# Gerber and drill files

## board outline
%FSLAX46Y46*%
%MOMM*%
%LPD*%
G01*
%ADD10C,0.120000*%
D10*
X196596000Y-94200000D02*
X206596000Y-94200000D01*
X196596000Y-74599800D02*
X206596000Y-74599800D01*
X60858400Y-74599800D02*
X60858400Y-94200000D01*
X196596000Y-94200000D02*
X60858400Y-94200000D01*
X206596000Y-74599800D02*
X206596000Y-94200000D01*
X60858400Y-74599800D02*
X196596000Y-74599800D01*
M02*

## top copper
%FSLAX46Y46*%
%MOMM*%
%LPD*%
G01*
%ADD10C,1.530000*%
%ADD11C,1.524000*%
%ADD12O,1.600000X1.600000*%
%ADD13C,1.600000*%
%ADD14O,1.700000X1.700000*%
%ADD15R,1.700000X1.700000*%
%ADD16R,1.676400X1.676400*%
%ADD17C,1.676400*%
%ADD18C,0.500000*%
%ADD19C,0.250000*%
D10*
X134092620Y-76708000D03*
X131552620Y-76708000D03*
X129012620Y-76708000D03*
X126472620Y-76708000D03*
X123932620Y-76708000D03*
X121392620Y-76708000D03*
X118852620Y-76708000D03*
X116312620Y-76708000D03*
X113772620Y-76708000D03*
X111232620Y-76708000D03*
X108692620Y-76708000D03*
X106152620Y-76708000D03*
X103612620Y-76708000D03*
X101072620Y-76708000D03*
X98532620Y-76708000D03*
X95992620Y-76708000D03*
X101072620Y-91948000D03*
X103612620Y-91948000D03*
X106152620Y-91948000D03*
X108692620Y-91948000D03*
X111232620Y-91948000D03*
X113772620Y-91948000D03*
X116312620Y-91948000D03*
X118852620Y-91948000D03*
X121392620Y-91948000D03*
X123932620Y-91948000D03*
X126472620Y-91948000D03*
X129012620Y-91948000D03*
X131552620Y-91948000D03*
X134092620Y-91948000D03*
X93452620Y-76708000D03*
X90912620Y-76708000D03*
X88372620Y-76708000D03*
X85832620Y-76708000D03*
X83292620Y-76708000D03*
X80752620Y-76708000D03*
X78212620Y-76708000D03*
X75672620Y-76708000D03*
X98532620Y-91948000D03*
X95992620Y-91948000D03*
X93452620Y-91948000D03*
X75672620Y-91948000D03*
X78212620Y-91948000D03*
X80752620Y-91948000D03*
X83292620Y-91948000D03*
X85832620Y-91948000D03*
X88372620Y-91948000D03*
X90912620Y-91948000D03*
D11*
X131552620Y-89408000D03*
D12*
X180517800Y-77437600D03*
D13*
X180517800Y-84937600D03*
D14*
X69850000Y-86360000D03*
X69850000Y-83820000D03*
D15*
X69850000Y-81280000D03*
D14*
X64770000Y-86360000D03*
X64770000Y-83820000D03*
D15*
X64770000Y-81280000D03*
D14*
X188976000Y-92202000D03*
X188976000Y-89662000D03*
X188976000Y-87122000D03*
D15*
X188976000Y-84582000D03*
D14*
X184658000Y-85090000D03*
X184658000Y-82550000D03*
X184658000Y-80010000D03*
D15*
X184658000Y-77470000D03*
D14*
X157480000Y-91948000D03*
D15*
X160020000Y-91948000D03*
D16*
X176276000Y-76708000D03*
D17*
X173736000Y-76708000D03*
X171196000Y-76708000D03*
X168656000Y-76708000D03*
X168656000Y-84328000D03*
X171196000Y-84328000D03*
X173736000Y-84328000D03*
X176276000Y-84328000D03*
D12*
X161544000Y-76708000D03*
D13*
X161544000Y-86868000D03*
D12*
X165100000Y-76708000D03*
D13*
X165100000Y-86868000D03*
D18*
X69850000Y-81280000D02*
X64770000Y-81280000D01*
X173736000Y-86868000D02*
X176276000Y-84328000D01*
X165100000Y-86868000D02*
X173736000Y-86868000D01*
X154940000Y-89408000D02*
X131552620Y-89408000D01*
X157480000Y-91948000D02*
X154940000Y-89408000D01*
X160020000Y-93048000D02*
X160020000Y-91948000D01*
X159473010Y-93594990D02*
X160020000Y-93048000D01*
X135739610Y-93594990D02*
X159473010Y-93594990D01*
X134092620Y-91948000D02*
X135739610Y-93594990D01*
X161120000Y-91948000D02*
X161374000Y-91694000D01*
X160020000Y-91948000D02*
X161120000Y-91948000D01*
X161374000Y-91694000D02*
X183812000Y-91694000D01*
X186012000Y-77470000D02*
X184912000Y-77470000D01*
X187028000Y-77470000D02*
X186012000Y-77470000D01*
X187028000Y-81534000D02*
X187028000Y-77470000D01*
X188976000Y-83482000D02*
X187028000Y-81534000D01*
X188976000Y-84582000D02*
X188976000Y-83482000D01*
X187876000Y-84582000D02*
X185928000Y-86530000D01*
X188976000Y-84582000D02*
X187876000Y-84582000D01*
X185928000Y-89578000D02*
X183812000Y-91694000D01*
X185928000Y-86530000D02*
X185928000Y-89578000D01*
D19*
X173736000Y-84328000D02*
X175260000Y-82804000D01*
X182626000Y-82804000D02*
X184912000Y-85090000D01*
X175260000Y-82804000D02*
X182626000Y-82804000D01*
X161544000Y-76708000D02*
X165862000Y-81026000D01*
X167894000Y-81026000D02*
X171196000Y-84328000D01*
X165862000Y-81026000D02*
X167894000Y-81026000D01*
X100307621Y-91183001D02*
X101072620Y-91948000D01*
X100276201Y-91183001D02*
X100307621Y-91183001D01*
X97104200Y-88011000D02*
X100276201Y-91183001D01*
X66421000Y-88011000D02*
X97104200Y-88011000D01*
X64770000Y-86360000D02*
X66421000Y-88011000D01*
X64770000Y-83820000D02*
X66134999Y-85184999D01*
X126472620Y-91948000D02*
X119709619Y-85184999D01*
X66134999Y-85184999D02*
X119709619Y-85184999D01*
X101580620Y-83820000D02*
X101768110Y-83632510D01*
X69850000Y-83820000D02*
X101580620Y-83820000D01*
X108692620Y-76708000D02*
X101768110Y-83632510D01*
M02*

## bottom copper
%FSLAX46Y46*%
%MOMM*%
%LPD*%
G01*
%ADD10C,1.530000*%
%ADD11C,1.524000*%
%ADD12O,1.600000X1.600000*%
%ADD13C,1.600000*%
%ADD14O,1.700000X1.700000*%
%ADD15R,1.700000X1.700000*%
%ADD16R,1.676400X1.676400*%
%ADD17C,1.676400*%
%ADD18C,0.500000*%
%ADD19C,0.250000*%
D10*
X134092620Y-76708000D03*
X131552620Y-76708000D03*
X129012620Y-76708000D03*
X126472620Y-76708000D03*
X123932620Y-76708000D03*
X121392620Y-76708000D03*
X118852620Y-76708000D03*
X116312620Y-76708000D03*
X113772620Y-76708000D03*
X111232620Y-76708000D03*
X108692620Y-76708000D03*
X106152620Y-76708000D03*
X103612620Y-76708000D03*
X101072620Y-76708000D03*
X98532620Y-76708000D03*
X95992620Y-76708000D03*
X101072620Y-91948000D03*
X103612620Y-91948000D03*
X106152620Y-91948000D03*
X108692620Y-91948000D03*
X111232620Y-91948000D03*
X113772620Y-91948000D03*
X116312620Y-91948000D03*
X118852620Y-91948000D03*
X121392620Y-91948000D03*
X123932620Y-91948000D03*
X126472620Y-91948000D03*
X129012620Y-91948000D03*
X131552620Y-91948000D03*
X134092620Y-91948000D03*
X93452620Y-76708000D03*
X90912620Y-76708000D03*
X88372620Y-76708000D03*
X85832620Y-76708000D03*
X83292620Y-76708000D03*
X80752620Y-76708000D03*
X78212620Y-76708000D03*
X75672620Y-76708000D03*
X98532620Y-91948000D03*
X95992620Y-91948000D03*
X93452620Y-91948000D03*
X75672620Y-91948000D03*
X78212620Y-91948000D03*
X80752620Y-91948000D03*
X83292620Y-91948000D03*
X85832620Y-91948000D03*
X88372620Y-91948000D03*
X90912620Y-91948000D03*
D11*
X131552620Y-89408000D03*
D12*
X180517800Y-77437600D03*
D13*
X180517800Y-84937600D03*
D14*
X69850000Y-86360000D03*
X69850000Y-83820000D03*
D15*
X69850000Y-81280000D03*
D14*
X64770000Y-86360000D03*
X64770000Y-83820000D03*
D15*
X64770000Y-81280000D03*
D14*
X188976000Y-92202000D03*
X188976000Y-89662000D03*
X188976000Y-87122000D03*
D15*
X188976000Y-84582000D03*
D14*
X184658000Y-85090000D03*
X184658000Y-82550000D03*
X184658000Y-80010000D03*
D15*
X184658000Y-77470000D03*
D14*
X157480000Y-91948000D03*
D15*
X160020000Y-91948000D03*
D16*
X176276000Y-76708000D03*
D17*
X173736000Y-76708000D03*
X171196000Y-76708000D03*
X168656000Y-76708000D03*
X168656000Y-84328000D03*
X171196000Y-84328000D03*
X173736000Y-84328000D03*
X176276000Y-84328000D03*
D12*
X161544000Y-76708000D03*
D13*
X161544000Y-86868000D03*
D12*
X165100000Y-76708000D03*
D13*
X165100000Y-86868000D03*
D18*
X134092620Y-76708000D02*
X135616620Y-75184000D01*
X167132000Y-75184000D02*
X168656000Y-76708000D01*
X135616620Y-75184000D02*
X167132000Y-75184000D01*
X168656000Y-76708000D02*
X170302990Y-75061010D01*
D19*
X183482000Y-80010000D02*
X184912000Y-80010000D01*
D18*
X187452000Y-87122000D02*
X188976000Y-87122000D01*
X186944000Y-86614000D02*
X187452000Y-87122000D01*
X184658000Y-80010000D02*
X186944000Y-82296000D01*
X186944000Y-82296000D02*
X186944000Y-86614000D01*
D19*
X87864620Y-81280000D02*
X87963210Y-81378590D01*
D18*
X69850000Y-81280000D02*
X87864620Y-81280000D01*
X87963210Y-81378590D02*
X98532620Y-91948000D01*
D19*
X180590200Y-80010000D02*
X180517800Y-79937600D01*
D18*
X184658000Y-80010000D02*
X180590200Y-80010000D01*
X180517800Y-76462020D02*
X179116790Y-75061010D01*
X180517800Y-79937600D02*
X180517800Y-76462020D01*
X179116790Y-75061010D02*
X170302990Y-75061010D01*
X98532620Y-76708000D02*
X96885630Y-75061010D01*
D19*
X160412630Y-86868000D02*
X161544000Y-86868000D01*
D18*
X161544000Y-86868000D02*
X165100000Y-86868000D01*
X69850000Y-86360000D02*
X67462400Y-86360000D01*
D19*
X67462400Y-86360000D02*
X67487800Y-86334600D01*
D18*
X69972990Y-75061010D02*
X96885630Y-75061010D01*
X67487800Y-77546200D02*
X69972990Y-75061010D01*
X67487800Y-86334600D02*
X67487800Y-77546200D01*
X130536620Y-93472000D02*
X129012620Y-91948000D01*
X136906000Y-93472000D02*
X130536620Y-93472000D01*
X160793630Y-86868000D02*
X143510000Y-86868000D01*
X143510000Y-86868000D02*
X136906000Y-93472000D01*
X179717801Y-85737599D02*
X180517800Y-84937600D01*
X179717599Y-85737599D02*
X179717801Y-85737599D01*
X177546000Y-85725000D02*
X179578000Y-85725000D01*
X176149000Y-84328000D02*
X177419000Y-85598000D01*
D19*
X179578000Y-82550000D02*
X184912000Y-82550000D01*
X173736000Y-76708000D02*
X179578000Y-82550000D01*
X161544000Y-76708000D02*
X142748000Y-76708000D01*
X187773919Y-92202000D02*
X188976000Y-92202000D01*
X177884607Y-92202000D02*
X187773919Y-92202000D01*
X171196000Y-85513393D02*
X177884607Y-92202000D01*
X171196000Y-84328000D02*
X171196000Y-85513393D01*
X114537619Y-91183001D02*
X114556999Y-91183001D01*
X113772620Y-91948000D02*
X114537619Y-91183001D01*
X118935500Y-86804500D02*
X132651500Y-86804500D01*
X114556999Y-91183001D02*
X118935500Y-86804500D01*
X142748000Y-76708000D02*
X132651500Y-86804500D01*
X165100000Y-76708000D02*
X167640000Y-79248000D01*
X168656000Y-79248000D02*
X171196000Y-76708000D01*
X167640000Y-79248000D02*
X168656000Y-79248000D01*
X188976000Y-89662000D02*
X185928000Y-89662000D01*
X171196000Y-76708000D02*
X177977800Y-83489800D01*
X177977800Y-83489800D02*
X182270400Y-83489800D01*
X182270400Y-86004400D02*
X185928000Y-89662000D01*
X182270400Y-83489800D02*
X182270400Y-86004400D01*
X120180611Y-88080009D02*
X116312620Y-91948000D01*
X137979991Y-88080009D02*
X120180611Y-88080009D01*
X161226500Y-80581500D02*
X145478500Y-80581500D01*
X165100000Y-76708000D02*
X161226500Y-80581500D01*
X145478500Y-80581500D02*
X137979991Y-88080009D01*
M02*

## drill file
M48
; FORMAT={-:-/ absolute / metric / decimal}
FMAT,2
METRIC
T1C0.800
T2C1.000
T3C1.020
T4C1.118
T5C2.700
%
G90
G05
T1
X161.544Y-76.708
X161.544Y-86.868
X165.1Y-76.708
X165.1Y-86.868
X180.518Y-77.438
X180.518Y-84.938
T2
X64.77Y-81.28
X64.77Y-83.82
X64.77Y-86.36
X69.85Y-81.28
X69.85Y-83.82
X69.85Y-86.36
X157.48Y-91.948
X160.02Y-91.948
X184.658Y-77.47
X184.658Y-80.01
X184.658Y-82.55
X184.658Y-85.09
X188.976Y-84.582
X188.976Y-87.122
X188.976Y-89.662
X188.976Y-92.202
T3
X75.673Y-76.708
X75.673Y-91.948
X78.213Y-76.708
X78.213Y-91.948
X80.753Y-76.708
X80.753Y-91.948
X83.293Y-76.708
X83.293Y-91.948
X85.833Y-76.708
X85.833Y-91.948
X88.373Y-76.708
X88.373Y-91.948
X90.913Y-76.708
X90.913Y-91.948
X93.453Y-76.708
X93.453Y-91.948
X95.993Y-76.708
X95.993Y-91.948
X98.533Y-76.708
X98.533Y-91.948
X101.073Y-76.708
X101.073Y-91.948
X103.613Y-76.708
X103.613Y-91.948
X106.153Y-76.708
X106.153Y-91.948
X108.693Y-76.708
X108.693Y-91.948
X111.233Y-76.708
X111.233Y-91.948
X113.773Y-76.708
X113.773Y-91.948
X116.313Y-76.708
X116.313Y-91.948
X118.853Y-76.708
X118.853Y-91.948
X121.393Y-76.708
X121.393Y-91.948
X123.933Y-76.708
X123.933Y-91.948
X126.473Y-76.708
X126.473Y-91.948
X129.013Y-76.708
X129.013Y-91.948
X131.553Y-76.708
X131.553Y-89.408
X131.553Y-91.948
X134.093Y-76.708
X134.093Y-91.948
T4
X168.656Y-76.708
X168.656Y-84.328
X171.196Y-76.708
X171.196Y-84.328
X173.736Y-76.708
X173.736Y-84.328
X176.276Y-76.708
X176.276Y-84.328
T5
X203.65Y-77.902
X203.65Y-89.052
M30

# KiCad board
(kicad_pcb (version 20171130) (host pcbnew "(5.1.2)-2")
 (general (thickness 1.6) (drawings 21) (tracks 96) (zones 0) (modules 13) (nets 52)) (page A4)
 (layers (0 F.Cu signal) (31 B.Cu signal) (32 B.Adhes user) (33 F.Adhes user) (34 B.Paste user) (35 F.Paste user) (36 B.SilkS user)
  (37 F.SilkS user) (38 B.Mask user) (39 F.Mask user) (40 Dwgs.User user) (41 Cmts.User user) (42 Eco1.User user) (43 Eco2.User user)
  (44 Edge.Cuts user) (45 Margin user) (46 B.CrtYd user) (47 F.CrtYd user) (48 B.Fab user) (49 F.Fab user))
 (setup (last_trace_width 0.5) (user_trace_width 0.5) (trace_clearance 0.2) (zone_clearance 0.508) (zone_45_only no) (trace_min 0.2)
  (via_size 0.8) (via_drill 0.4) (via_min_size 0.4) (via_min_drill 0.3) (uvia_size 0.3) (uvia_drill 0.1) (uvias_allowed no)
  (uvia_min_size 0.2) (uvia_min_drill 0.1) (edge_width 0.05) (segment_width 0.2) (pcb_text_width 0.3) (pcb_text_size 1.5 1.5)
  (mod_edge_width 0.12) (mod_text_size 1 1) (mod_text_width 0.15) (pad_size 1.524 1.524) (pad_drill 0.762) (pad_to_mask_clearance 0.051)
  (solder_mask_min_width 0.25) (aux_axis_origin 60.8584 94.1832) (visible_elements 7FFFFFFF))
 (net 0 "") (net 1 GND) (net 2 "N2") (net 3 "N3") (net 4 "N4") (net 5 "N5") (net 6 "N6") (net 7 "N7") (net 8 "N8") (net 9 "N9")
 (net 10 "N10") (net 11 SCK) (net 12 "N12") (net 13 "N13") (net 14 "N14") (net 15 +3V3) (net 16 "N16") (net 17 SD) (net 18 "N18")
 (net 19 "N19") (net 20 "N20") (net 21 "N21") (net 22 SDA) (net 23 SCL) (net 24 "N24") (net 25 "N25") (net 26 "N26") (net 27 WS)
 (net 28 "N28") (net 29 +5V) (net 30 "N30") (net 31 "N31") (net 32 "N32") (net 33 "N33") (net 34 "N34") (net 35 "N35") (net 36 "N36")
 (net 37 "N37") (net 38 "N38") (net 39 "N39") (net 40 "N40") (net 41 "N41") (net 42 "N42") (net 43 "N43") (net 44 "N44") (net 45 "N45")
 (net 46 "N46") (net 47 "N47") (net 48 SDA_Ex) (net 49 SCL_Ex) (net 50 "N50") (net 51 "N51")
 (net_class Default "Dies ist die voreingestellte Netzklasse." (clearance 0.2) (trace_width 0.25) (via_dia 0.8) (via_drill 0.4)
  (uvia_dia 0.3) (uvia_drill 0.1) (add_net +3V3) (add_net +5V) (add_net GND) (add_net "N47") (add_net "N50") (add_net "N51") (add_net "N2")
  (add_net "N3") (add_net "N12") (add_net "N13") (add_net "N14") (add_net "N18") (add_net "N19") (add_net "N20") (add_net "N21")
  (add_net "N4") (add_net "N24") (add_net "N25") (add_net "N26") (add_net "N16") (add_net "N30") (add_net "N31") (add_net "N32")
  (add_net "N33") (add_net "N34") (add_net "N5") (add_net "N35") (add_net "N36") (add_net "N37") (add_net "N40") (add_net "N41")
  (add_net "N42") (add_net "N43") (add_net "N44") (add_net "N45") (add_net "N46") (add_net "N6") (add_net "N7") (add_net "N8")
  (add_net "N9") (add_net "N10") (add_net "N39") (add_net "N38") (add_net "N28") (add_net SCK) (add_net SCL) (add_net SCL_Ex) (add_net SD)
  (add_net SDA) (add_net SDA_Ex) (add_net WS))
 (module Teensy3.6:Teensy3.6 (layer F.Cu) (at 104.88262 84.328 270)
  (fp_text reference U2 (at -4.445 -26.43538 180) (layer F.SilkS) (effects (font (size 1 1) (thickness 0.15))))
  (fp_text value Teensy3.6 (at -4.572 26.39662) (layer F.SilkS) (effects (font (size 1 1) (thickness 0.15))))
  (pad GND_1 thru_hole circle (at -7.62 -29.21 270) (size 1.53 1.53) (drill 1.02) (layers *.Cu *.Mask) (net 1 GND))
  (pad 0 thru_hole circle (at -7.62 -26.67 270) (size 1.53 1.53) (drill 1.02) (layers *.Cu *.Mask) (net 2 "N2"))
  (pad 1 thru_hole circle (at -7.62 -24.13 270) (size 1.53 1.53) (drill 1.02) (layers *.Cu *.Mask) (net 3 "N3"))
  (pad 2 thru_hole circle (at -7.62 -21.59 270) (size 1.53 1.53) (drill 1.02) (layers *.Cu *.Mask) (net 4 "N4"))
  (pad 3 thru_hole circle (at -7.62 -19.05 270) (size 1.53 1.53) (drill 1.02) (layers *.Cu *.Mask) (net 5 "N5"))
  (pad 4 thru_hole circle (at -7.62 -16.51 270) (size 1.53 1.53) (drill 1.02) (layers *.Cu *.Mask) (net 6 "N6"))
  (pad 5 thru_hole circle (at -7.62 -13.97 270) (size 1.53 1.53) (drill 1.02) (layers *.Cu *.Mask) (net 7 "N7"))
  (pad 6 thru_hole circle (at -7.62 -11.43 270) (size 1.53 1.53) (drill 1.02) (layers *.Cu *.Mask) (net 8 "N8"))
  (pad 7 thru_hole circle (at -7.62 -8.89 270) (size 1.53 1.53) (drill 1.02) (layers *.Cu *.Mask) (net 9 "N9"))
  (pad 8 thru_hole circle (at -7.62 -6.35 270) (size 1.53 1.53) (drill 1.02) (layers *.Cu *.Mask) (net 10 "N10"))
  (pad 9 thru_hole circle (at -7.62 -3.81 270) (size 1.53 1.53) (drill 1.02) (layers *.Cu *.Mask) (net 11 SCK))
  (pad 10 thru_hole circle (at -7.62 -1.27 270) (size 1.53 1.53) (drill 1.02) (layers *.Cu *.Mask) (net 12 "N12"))
  (pad 11 thru_hole circle (at -7.62 1.27 270) (size 1.53 1.53) (drill 1.02) (layers *.Cu *.Mask) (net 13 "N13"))
  (pad 12 thru_hole circle (at -7.62 3.81 270) (size 1.53 1.53) (drill 1.02) (layers *.Cu *.Mask) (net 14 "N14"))
  (pad 3V3_1 thru_hole circle (at -7.62 6.35 270) (size 1.53 1.53) (drill 1.02) (layers *.Cu *.Mask) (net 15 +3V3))
  (pad 24 thru_hole circle (at -7.62 8.89 270) (size 1.53 1.53) (drill 1.02) (layers *.Cu *.Mask) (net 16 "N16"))
  (pad 13 thru_hole circle (at 7.62 3.81 270) (size 1.53 1.53) (drill 1.02) (layers *.Cu *.Mask) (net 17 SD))
  (pad 14 thru_hole circle (at 7.62 1.27 270) (size 1.53 1.53) (drill 1.02) (layers *.Cu *.Mask) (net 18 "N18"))
  (pad 15 thru_hole circle (at 7.62 -1.27 270) (size 1.53 1.53) (drill 1.02) (layers *.Cu *.Mask) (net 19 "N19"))
  (pad 16 thru_hole circle (at 7.62 -3.81 270) (size 1.53 1.53) (drill 1.02) (layers *.Cu *.Mask) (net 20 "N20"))
  (pad 17 thru_hole circle (at 7.62 -6.35 270) (size 1.53 1.53) (drill 1.02) (layers *.Cu *.Mask) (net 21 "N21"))
  (pad 18 thru_hole circle (at 7.62 -8.89 270) (size 1.53 1.53) (drill 1.02) (layers *.Cu *.Mask) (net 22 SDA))
  (pad 19 thru_hole circle (at 7.62 -11.43 270) (size 1.53 1.53) (drill 1.02) (layers *.Cu *.Mask) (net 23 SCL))
  (pad 20 thru_hole circle (at 7.62 -13.97 270) (size 1.53 1.53) (drill 1.02) (layers *.Cu *.Mask) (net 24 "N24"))
  (pad 21 thru_hole circle (at 7.62 -16.51 270) (size 1.53 1.53) (drill 1.02) (layers *.Cu *.Mask) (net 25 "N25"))
  (pad 22 thru_hole circle (at 7.62 -19.05 270) (size 1.53 1.53) (drill 1.02) (layers *.Cu *.Mask) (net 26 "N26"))
  (pad 23 thru_hole circle (at 7.62 -21.59 270) (size 1.53 1.53) (drill 1.02) (layers *.Cu *.Mask) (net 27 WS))
  (pad 3V3_2 thru_hole circle (at 7.62 -24.13 270) (size 1.53 1.53) (drill 1.02) (layers *.Cu *.Mask) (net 15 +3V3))
  (pad AGND thru_hole circle (at 7.62 -26.67 270) (size 1.53 1.53) (drill 1.02) (layers *.Cu *.Mask) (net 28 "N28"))
  (pad VIN thru_hole circle (at 7.62 -29.21 270) (size 1.53 1.53) (drill 1.02) (layers *.Cu *.Mask) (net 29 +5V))
  (pad 25 thru_hole circle (at -7.62 11.43 270) (size 1.53 1.53) (drill 1.02) (layers *.Cu *.Mask) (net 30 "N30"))
  (pad 26 thru_hole circle (at -7.62 13.97 270) (size 1.53 1.53) (drill 1.02) (layers *.Cu *.Mask) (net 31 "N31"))
  (pad 27 thru_hole circle (at -7.62 16.51 270) (size 1.53 1.53) (drill 1.02) (layers *.Cu *.Mask) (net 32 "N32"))
  (pad 28 thru_hole circle (at -7.62 19.05 270) (size 1.53 1.53) (drill 1.02) (layers *.Cu *.Mask) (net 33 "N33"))
  (pad 29 thru_hole circle (at -7.62 21.59 270) (size 1.53 1.53) (drill 1.02) (layers *.Cu *.Mask) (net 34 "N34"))
  (pad 30 thru_hole circle (at -7.62 24.13 270) (size 1.53 1.53) (drill 1.02) (layers *.Cu *.Mask) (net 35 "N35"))
  (pad 31 thru_hole circle (at -7.62 26.67 270) (size 1.53 1.53) (drill 1.02) (layers *.Cu *.Mask) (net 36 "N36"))
  (pad 32 thru_hole circle (at -7.62 29.21 270) (size 1.53 1.53) (drill 1.02) (layers *.Cu *.Mask) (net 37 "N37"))
  (pad GND_2 thru_hole circle (at 7.62 6.35 270) (size 1.53 1.53) (drill 1.02) (layers *.Cu *.Mask) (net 1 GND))
  (pad A22 thru_hole circle (at 7.62 8.89 270) (size 1.53 1.53) (drill 1.02) (layers *.Cu *.Mask) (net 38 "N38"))
  (pad A21 thru_hole circle (at 7.62 11.43 270) (size 1.53 1.53) (drill 1.02) (layers *.Cu *.Mask) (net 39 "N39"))
  (pad 33 thru_hole circle (at 7.62 29.21 270) (size 1.53 1.53) (drill 1.02) (layers *.Cu *.Mask) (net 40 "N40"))
  (pad 34 thru_hole circle (at 7.62 26.67 270) (size 1.53 1.53) (drill 1.02) (layers *.Cu *.Mask) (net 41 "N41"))
  (pad 35 thru_hole circle (at 7.62 24.13 270) (size 1.53 1.53) (drill 1.02) (layers *.Cu *.Mask) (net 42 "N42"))
  (pad 36 thru_hole circle (at 7.62 21.59 270) (size 1.53 1.53) (drill 1.02) (layers *.Cu *.Mask) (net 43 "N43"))
  (pad 37 thru_hole circle (at 7.62 19.05 270) (size 1.53 1.53) (drill 1.02) (layers *.Cu *.Mask) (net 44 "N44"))
  (pad 38 thru_hole circle (at 7.62 16.51 270) (size 1.53 1.53) (drill 1.02) (layers *.Cu *.Mask) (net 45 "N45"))
  (pad 39 thru_hole circle (at 7.62 13.97 270) (size 1.53 1.53) (drill 1.02) (layers *.Cu *.Mask) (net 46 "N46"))
  (pad VUSB thru_hole circle (at 5.08 -26.67 270) (size 1.524 1.524) (drill 1.02) (layers *.Cu *.Mask) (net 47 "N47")))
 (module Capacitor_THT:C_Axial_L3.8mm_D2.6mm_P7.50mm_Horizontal (layer F.Cu) (at 180.5178 84.9376 90)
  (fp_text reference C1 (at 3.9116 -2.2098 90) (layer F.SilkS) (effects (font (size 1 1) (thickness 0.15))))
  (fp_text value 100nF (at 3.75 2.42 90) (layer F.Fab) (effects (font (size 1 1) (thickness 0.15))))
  (pad 2 thru_hole oval (at 7.5 0 90) (size 1.6 1.6) (drill 0.8) (layers *.Cu *.Mask) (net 1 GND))
  (pad 1 thru_hole circle (at 0 0 90) (size 1.6 1.6) (drill 0.8) (layers *.Cu *.Mask) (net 15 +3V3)))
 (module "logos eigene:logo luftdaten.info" (layer F.Cu) (at 143.1798 88.5698)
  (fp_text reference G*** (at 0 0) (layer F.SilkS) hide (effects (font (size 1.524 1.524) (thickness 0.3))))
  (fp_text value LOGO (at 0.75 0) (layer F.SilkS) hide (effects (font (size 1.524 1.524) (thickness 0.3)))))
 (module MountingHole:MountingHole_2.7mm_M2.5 (layer F.Cu) (at 203.6496 89.0524)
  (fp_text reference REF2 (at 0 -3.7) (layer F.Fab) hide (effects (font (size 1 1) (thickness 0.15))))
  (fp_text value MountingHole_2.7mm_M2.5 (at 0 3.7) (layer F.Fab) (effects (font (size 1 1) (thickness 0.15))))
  (pad 1 np_thru_hole circle (at 0 0) (size 2.7 2.7) (drill 2.7) (layers *.Cu *.Mask)))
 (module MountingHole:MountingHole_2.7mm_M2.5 (layer F.Cu) (at 203.6496 77.9018)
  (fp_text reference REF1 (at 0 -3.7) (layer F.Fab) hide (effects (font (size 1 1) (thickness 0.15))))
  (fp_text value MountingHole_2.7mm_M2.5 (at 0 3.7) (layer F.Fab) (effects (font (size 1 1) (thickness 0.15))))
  (pad 1 np_thru_hole circle (at 0 0) (size 2.7 2.7) (drill 2.7) (layers *.Cu *.Mask)))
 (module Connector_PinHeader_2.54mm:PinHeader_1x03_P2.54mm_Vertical (layer F.Cu) (at 69.85 81.28)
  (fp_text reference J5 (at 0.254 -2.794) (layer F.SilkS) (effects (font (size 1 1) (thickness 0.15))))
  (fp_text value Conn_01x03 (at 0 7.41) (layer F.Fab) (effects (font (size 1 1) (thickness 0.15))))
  (pad 3 thru_hole oval (at 0 5.08) (size 1.7 1.7) (drill 1) (layers *.Cu *.Mask) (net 15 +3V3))
  (pad 2 thru_hole oval (at 0 2.54) (size 1.7 1.7) (drill 1) (layers *.Cu *.Mask) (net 11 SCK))
  (pad 1 thru_hole rect (at 0 0) (size 1.7 1.7) (drill 1) (layers *.Cu *.Mask) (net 1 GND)))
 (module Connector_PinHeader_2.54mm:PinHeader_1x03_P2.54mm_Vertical (layer F.Cu) (at 64.77 81.28)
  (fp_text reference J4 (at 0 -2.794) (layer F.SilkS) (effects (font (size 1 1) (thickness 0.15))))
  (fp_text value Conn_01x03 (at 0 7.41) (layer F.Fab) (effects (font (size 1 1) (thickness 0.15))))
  (pad 3 thru_hole oval (at 0 5.08) (size 1.7 1.7) (drill 1) (layers *.Cu *.Mask) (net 17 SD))
  (pad 2 thru_hole oval (at 0 2.54) (size 1.7 1.7) (drill 1) (layers *.Cu *.Mask) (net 27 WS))
  (pad 1 thru_hole rect (at 0 0) (size 1.7 1.7) (drill 1) (layers *.Cu *.Mask) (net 1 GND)))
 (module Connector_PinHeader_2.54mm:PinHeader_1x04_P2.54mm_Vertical (layer F.Cu) (at 188.976 84.582)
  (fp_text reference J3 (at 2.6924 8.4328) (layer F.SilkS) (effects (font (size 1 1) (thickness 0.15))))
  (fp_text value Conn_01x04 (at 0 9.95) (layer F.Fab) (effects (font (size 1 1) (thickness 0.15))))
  (pad 4 thru_hole oval (at 0 7.62) (size 1.7 1.7) (drill 1) (layers *.Cu *.Mask) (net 22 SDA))
  (pad 3 thru_hole oval (at 0 5.08) (size 1.7 1.7) (drill 1) (layers *.Cu *.Mask) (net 23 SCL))
  (pad 2 thru_hole oval (at 0 2.54) (size 1.7 1.7) (drill 1) (layers *.Cu *.Mask) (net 1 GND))
  (pad 1 thru_hole rect (at 0 0) (size 1.7 1.7) (drill 1) (layers *.Cu *.Mask) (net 29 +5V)))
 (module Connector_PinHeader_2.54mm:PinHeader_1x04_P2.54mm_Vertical (layer F.Cu) (at 184.658 77.47)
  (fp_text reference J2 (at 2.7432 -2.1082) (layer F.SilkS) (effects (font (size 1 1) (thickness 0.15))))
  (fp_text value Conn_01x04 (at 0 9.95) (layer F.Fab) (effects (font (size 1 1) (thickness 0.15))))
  (pad 4 thru_hole oval (at 0 7.62) (size 1.7 1.7) (drill 1) (layers *.Cu *.Mask) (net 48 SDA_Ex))
  (pad 3 thru_hole oval (at 0 5.08) (size 1.7 1.7) (drill 1) (layers *.Cu *.Mask) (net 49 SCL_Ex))
  (pad 2 thru_hole oval (at 0 2.54) (size 1.7 1.7) (drill 1) (layers *.Cu *.Mask) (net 1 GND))
  (pad 1 thru_hole rect (at 0 0) (size 1.7 1.7) (drill 1) (layers *.Cu *.Mask) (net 29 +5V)))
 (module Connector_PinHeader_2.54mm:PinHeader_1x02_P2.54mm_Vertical (layer F.Cu) (at 160.02 91.948 270)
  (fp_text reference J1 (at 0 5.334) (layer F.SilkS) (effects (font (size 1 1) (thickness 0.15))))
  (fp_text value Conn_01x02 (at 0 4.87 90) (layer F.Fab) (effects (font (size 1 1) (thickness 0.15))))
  (pad 2 thru_hole oval (at 0 2.54 270) (size 1.7 1.7) (drill 1) (layers *.Cu *.Mask) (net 47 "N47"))
  (pad 1 thru_hole rect (at 0 0 270) (size 1.7 1.7) (drill 1) (layers *.Cu *.Mask) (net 29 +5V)))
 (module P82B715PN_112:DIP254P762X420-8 (layer F.Cu) (at 168.656 84.328 270)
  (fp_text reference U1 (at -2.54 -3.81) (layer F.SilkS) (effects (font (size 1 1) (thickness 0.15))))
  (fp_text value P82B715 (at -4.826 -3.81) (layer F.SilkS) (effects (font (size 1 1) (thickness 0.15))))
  (pad 1 thru_hole rect (at -7.62 -7.62 270) (size 1.6764 1.6764) (drill 1.1176) (layers *.Cu *.Mask) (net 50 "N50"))
  (pad 2 thru_hole circle (at -7.62 -5.08 270) (size 1.6764 1.6764) (drill 1.1176) (layers *.Cu *.Mask) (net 49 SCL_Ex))
  (pad 3 thru_hole circle (at -7.62 -2.54 270) (size 1.6764 1.6764) (drill 1.1176) (layers *.Cu *.Mask) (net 23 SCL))
  (pad 4 thru_hole circle (at -7.62 0 270) (size 1.6764 1.6764) (drill 1.1176) (layers *.Cu *.Mask) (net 1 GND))
  (pad 5 thru_hole circle (at 0 0 270) (size 1.6764 1.6764) (drill 1.1176) (layers *.Cu *.Mask) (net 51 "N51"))
  (pad 6 thru_hole circle (at 0 -2.54 270) (size 1.6764 1.6764) (drill 1.1176) (layers *.Cu *.Mask) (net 22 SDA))
  (pad 7 thru_hole circle (at 0 -5.08 270) (size 1.6764 1.6764) (drill 1.1176) (layers *.Cu *.Mask) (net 48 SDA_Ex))
  (pad 8 thru_hole circle (at 0 -7.62 270) (size 1.6764 1.6764) (drill 1.1176) (layers *.Cu *.Mask) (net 15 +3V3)))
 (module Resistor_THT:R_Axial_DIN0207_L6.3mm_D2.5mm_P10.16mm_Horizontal (layer F.Cu) (at 161.544 86.868 90)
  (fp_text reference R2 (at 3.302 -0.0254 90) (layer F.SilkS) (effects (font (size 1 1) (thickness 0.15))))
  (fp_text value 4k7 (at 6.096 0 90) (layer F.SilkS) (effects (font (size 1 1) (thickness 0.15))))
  (pad 2 thru_hole oval (at 10.16 0 90) (size 1.6 1.6) (drill 0.8) (layers *.Cu *.Mask) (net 22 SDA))
  (pad 1 thru_hole circle (at 0 0 90) (size 1.6 1.6) (drill 0.8) (layers *.Cu *.Mask) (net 15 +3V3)))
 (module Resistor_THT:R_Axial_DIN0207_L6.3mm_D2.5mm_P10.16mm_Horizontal (layer F.Cu) (at 165.1 86.868 90)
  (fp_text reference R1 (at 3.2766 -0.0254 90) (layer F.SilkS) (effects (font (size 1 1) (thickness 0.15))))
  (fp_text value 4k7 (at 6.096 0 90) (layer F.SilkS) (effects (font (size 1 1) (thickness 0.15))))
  (pad 2 thru_hole oval (at 10.16 0 90) (size 1.6 1.6) (drill 0.8) (layers *.Cu *.Mask) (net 23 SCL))
  (pad 1 thru_hole circle (at 0 0 90) (size 1.6 1.6) (drill 0.8) (layers *.Cu *.Mask) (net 15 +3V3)))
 (gr_line (start 196.596 94.2) (end 206.596 94.2) (layer Edge.Cuts) (width 0.12))
 (gr_line (start 196.596 74.5998) (end 206.596 74.5998) (layer Edge.Cuts) (width 0.12))
 (gr_line (start 60.8584 74.5998) (end 60.8584 94.2) (layer Edge.Cuts) (width 0.12))
 (gr_line (start 196.596 94.2) (end 60.8584 94.2) (layer Edge.Cuts) (width 0.12))
 (gr_line (start 206.596 74.5998) (end 206.596 94.2) (layer Edge.Cuts) (width 0.12))
 (gr_line (start 60.8584 74.5998) (end 196.596 74.5998) (layer Edge.Cuts) (width 0.12))
 (segment (start 134.09262 76.708) (end 135.61662 75.184) (width 0.5) (layer B.Cu) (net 1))
 (segment (start 167.132 75.184) (end 168.656 76.708) (width 0.5) (layer B.Cu) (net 1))
 (segment (start 135.61662 75.184) (end 167.132 75.184) (width 0.5) (layer B.Cu) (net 1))
 (segment (start 168.656 76.708) (end 170.30299 75.06101) (width 0.5) (layer B.Cu) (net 1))
 (segment (start 183.482 80.01) (end 184.912 80.01) (width 0.25) (layer B.Cu) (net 1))
 (segment (start 187.452 87.122) (end 188.976 87.122) (width 0.5) (layer B.Cu) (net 1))
 (segment (start 186.944 86.614) (end 187.452 87.122) (width 0.5) (layer B.Cu) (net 1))
 (segment (start 184.658 80.01) (end 186.944 82.296) (width 0.5) (layer B.Cu) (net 1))
 (segment (start 186.944 82.296) (end 186.944 86.614) (width 0.5) (layer B.Cu) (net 1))
 (segment (start 87.86462 81.28) (end 87.96321 81.37859) (width 0.25) (layer B.Cu) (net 1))
 (segment (start 69.85 81.28) (end 87.86462 81.28) (width 0.5) (layer B.Cu) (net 1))
 (segment (start 87.96321 81.37859) (end 98.53262 91.948) (width 0.5) (layer B.Cu) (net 1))
 (segment (start 69.85 81.28) (end 64.77 81.28) (width 0.5) (layer F.Cu) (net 1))
 (segment (start 180.5902 80.01) (end 180.5178 79.9376) (width 0.25) (layer B.Cu) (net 1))
 (segment (start 184.658 80.01) (end 180.5902 80.01) (width 0.5) (layer B.Cu) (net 1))
 (segment (start 180.5178 76.46202) (end 179.11679 75.06101) (width 0.5) (layer B.Cu) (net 1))
 (segment (start 180.5178 79.9376) (end 180.5178 76.46202) (width 0.5) (layer B.Cu) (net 1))
 (segment (start 179.11679 75.06101) (end 170.30299 75.06101) (width 0.5) (layer B.Cu) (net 1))
 (segment (start 98.53262 76.708) (end 96.88563 75.06101) (width 0.5) (layer B.Cu) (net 15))
 (segment (start 160.41263 86.868) (end 161.544 86.868) (width 0.25) (layer B.Cu) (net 15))
 (segment (start 161.544 86.868) (end 165.1 86.868) (width 0.5) (layer B.Cu) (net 15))
 (segment (start 173.736 86.868) (end 176.276 84.328) (width 0.5) (layer F.Cu) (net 15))
 (segment (start 165.1 86.868) (end 173.736 86.868) (width 0.5) (layer F.Cu) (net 15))
 (segment (start 69.85 86.36) (end 67.4624 86.36) (width 0.5) (layer B.Cu) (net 15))
 (segment (start 67.4624 86.36) (end 67.4878 86.3346) (width 0.25) (layer B.Cu) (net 15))
 (segment (start 69.97299 75.06101) (end 96.88563 75.06101) (width 0.5) (layer B.Cu) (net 15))
 (segment (start 67.4878 77.5462) (end 69.97299 75.06101) (width 0.5) (layer B.Cu) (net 15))
 (segment (start 67.4878 86.3346) (end 67.4878 77.5462) (width 0.5) (layer B.Cu) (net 15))
 (segment (start 130.53662 93.472) (end 129.01262 91.948) (width 0.5) (layer B.Cu) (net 15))
 (segment (start 136.906 93.472) (end 130.53662 93.472) (width 0.5) (layer B.Cu) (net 15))
 (segment (start 160.79363 86.868) (end 143.51 86.868) (width 0.5) (layer B.Cu) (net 15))
 (segment (start 143.51 86.868) (end 136.906 93.472) (width 0.5) (layer B.Cu) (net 15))
 (segment (start 179.717801 85.737599) (end 180.5178 84.9376) (width 0.5) (layer B.Cu) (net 15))
 (segment (start 179.717599 85.737599) (end 179.717801 85.737599) (width 0.5) (layer B.Cu) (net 15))
 (segment (start 177.546 85.725) (end 179.578 85.725) (width 0.5) (layer B.Cu) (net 15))
 (segment (start 176.149 84.328) (end 177.419 85.598) (width 0.5) (layer B.Cu) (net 15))
 (segment (start 154.94 89.408) (end 131.55262 89.408) (width 0.5) (layer F.Cu) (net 47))
 (segment (start 157.48 91.948) (end 154.94 89.408) (width 0.5) (layer F.Cu) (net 47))
 (segment (start 160.02 93.048) (end 160.02 91.948) (width 0.5) (layer F.Cu) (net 29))
 (segment (start 159.47301 93.59499) (end 160.02 93.048) (width 0.5) (layer F.Cu) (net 29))
 (segment (start 135.73961 93.59499) (end 159.47301 93.59499) (width 0.5) (layer F.Cu) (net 29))
 (segment (start 134.09262 91.948) (end 135.73961 93.59499) (width 0.5) (layer F.Cu) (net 29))
 (segment (start 161.12 91.948) (end 161.374 91.694) (width 0.5) (layer F.Cu) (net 29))
 (segment (start 160.02 91.948) (end 161.12 91.948) (width 0.5) (layer F.Cu) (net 29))
 (segment (start 161.374 91.694) (end 183.812 91.694) (width 0.5) (layer F.Cu) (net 29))
 (segment (start 186.012 77.47) (end 184.912 77.47) (width 0.5) (layer F.Cu) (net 29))
 (segment (start 187.028 77.47) (end 186.012 77.47) (width 0.5) (layer F.Cu) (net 29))
 (segment (start 187.028 81.534) (end 187.028 77.47) (width 0.5) (layer F.Cu) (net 29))
 (segment (start 188.976 83.482) (end 187.028 81.534) (width 0.5) (layer F.Cu) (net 29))
 (segment (start 188.976 84.582) (end 188.976 83.482) (width 0.5) (layer F.Cu) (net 29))
 (segment (start 187.876 84.582) (end 185.928 86.53) (width 0.5) (layer F.Cu) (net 29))
 (segment (start 188.976 84.582) (end 187.876 84.582) (width 0.5) (layer F.Cu) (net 29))
 (segment (start 185.928 89.578) (end 183.812 91.694) (width 0.5) (layer F.Cu) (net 29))
 (segment (start 185.928 86.53) (end 185.928 89.578) (width 0.5) (layer F.Cu) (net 29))
 (segment (start 173.736 84.328) (end 175.26 82.804) (width 0.25) (layer F.Cu) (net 48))
 (segment (start 182.626 82.804) (end 184.912 85.09) (width 0.25) (layer F.Cu) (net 48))
 (segment (start 175.26 82.804) (end 182.626 82.804) (width 0.25) (layer F.Cu) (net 48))
 (segment (start 179.578 82.55) (end 184.912 82.55) (width 0.25) (layer B.Cu) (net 49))
 (segment (start 173.736 76.708) (end 179.578 82.55) (width 0.25) (layer B.Cu) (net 49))
 (segment (start 161.544 76.708) (end 142.748 76.708) (width 0.25) (layer B.Cu) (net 22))
 (segment (start 161.544 76.708) (end 165.862 81.026) (width 0.25) (layer F.Cu) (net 22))
 (segment (start 167.894 81.026) (end 171.196 84.328) (width 0.25) (layer F.Cu) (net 22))
 (segment (start 165.862 81.026) (end 167.894 81.026) (width 0.25) (layer F.Cu) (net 22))
 (segment (start 187.773919 92.202) (end 188.976 92.202) (width 0.25) (layer B.Cu) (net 22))
 (segment (start 177.884607 92.202) (end 187.773919 92.202) (width 0.25) (layer B.Cu) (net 22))
 (segment (start 171.196 85.513393) (end 177.884607 92.202) (width 0.25) (layer B.Cu) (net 22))
 (segment (start 171.196 84.328) (end 171.196 85.513393) (width 0.25) (layer B.Cu) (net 22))
 (segment (start 114.537619 91.183001) (end 114.556999 91.183001) (width 0.25) (layer B.Cu) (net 22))
 (segment (start 113.77262 91.948) (end 114.537619 91.183001) (width 0.25) (layer B.Cu) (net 22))
 (segment (start 118.9355 86.8045) (end 132.6515 86.8045) (width 0.25) (layer B.Cu) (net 22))
 (segment (start 114.556999 91.183001) (end 118.9355 86.8045) (width 0.25) (layer B.Cu) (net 22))
 (segment (start 142.748 76.708) (end 132.6515 86.8045) (width 0.25) (layer B.Cu) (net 22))
 (segment (start 165.1 76.708) (end 167.64 79.248) (width 0.25) (layer B.Cu) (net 23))
 (segment (start 168.656 79.248) (end 171.196 76.708) (width 0.25) (layer B.Cu) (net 23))
 (segment (start 167.64 79.248) (end 168.656 79.248) (width 0.25) (layer B.Cu) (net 23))
 (segment (start 188.976 89.662) (end 185.928 89.662) (width 0.25) (layer B.Cu) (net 23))
 (segment (start 171.196 76.708) (end 177.9778 83.4898) (width 0.25) (layer B.Cu) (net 23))
 (segment (start 177.9778 83.4898) (end 182.2704 83.4898) (width 0.25) (layer B.Cu) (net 23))
 (segment (start 182.2704 86.0044) (end 185.928 89.662) (width 0.25) (layer B.Cu) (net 23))
 (segment (start 182.2704 83.4898) (end 182.2704 86.0044) (width 0.25) (layer B.Cu) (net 23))
 (segment (start 120.180611 88.080009) (end 116.31262 91.948) (width 0.25) (layer B.Cu) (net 23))
 (segment (start 137.979991 88.080009) (end 120.180611 88.080009) (width 0.25) (layer B.Cu) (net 23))
 (segment (start 161.2265 80.5815) (end 145.4785 80.5815) (width 0.25) (layer B.Cu) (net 23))
 (segment (start 165.1 76.708) (end 161.2265 80.5815) (width 0.25) (layer B.Cu) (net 23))
 (segment (start 145.4785 80.5815) (end 137.979991 88.080009) (width 0.25) (layer B.Cu) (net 23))
 (segment (start 100.307621 91.183001) (end 101.07262 91.948) (width 0.25) (layer F.Cu) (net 17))
 (segment (start 100.276201 91.183001) (end 100.307621 91.183001) (width 0.25) (layer F.Cu) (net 17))
 (segment (start 97.1042 88.011) (end 100.276201 91.183001) (width 0.25) (layer F.Cu) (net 17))
 (segment (start 66.421 88.011) (end 97.1042 88.011) (width 0.25) (layer F.Cu) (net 17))
 (segment (start 64.77 86.36) (end 66.421 88.011) (width 0.25) (layer F.Cu) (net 17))
 (segment (start 64.77 83.82) (end 66.134999 85.184999) (width 0.25) (layer F.Cu) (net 27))
 (segment (start 126.47262 91.948) (end 119.709619 85.184999) (width 0.25) (layer F.Cu) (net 27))
 (segment (start 66.134999 85.184999) (end 119.709619 85.184999) (width 0.25) (layer F.Cu) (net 27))
 (segment (start 101.58062 83.82) (end 101.76811 83.63251) (width 0.25) (layer F.Cu) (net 11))
 (segment (start 69.85 83.82) (end 101.58062 83.82) (width 0.25) (layer F.Cu) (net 11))
 (segment (start 108.69262 76.708) (end 101.76811 83.63251) (width 0.25) (layer F.Cu) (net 11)))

